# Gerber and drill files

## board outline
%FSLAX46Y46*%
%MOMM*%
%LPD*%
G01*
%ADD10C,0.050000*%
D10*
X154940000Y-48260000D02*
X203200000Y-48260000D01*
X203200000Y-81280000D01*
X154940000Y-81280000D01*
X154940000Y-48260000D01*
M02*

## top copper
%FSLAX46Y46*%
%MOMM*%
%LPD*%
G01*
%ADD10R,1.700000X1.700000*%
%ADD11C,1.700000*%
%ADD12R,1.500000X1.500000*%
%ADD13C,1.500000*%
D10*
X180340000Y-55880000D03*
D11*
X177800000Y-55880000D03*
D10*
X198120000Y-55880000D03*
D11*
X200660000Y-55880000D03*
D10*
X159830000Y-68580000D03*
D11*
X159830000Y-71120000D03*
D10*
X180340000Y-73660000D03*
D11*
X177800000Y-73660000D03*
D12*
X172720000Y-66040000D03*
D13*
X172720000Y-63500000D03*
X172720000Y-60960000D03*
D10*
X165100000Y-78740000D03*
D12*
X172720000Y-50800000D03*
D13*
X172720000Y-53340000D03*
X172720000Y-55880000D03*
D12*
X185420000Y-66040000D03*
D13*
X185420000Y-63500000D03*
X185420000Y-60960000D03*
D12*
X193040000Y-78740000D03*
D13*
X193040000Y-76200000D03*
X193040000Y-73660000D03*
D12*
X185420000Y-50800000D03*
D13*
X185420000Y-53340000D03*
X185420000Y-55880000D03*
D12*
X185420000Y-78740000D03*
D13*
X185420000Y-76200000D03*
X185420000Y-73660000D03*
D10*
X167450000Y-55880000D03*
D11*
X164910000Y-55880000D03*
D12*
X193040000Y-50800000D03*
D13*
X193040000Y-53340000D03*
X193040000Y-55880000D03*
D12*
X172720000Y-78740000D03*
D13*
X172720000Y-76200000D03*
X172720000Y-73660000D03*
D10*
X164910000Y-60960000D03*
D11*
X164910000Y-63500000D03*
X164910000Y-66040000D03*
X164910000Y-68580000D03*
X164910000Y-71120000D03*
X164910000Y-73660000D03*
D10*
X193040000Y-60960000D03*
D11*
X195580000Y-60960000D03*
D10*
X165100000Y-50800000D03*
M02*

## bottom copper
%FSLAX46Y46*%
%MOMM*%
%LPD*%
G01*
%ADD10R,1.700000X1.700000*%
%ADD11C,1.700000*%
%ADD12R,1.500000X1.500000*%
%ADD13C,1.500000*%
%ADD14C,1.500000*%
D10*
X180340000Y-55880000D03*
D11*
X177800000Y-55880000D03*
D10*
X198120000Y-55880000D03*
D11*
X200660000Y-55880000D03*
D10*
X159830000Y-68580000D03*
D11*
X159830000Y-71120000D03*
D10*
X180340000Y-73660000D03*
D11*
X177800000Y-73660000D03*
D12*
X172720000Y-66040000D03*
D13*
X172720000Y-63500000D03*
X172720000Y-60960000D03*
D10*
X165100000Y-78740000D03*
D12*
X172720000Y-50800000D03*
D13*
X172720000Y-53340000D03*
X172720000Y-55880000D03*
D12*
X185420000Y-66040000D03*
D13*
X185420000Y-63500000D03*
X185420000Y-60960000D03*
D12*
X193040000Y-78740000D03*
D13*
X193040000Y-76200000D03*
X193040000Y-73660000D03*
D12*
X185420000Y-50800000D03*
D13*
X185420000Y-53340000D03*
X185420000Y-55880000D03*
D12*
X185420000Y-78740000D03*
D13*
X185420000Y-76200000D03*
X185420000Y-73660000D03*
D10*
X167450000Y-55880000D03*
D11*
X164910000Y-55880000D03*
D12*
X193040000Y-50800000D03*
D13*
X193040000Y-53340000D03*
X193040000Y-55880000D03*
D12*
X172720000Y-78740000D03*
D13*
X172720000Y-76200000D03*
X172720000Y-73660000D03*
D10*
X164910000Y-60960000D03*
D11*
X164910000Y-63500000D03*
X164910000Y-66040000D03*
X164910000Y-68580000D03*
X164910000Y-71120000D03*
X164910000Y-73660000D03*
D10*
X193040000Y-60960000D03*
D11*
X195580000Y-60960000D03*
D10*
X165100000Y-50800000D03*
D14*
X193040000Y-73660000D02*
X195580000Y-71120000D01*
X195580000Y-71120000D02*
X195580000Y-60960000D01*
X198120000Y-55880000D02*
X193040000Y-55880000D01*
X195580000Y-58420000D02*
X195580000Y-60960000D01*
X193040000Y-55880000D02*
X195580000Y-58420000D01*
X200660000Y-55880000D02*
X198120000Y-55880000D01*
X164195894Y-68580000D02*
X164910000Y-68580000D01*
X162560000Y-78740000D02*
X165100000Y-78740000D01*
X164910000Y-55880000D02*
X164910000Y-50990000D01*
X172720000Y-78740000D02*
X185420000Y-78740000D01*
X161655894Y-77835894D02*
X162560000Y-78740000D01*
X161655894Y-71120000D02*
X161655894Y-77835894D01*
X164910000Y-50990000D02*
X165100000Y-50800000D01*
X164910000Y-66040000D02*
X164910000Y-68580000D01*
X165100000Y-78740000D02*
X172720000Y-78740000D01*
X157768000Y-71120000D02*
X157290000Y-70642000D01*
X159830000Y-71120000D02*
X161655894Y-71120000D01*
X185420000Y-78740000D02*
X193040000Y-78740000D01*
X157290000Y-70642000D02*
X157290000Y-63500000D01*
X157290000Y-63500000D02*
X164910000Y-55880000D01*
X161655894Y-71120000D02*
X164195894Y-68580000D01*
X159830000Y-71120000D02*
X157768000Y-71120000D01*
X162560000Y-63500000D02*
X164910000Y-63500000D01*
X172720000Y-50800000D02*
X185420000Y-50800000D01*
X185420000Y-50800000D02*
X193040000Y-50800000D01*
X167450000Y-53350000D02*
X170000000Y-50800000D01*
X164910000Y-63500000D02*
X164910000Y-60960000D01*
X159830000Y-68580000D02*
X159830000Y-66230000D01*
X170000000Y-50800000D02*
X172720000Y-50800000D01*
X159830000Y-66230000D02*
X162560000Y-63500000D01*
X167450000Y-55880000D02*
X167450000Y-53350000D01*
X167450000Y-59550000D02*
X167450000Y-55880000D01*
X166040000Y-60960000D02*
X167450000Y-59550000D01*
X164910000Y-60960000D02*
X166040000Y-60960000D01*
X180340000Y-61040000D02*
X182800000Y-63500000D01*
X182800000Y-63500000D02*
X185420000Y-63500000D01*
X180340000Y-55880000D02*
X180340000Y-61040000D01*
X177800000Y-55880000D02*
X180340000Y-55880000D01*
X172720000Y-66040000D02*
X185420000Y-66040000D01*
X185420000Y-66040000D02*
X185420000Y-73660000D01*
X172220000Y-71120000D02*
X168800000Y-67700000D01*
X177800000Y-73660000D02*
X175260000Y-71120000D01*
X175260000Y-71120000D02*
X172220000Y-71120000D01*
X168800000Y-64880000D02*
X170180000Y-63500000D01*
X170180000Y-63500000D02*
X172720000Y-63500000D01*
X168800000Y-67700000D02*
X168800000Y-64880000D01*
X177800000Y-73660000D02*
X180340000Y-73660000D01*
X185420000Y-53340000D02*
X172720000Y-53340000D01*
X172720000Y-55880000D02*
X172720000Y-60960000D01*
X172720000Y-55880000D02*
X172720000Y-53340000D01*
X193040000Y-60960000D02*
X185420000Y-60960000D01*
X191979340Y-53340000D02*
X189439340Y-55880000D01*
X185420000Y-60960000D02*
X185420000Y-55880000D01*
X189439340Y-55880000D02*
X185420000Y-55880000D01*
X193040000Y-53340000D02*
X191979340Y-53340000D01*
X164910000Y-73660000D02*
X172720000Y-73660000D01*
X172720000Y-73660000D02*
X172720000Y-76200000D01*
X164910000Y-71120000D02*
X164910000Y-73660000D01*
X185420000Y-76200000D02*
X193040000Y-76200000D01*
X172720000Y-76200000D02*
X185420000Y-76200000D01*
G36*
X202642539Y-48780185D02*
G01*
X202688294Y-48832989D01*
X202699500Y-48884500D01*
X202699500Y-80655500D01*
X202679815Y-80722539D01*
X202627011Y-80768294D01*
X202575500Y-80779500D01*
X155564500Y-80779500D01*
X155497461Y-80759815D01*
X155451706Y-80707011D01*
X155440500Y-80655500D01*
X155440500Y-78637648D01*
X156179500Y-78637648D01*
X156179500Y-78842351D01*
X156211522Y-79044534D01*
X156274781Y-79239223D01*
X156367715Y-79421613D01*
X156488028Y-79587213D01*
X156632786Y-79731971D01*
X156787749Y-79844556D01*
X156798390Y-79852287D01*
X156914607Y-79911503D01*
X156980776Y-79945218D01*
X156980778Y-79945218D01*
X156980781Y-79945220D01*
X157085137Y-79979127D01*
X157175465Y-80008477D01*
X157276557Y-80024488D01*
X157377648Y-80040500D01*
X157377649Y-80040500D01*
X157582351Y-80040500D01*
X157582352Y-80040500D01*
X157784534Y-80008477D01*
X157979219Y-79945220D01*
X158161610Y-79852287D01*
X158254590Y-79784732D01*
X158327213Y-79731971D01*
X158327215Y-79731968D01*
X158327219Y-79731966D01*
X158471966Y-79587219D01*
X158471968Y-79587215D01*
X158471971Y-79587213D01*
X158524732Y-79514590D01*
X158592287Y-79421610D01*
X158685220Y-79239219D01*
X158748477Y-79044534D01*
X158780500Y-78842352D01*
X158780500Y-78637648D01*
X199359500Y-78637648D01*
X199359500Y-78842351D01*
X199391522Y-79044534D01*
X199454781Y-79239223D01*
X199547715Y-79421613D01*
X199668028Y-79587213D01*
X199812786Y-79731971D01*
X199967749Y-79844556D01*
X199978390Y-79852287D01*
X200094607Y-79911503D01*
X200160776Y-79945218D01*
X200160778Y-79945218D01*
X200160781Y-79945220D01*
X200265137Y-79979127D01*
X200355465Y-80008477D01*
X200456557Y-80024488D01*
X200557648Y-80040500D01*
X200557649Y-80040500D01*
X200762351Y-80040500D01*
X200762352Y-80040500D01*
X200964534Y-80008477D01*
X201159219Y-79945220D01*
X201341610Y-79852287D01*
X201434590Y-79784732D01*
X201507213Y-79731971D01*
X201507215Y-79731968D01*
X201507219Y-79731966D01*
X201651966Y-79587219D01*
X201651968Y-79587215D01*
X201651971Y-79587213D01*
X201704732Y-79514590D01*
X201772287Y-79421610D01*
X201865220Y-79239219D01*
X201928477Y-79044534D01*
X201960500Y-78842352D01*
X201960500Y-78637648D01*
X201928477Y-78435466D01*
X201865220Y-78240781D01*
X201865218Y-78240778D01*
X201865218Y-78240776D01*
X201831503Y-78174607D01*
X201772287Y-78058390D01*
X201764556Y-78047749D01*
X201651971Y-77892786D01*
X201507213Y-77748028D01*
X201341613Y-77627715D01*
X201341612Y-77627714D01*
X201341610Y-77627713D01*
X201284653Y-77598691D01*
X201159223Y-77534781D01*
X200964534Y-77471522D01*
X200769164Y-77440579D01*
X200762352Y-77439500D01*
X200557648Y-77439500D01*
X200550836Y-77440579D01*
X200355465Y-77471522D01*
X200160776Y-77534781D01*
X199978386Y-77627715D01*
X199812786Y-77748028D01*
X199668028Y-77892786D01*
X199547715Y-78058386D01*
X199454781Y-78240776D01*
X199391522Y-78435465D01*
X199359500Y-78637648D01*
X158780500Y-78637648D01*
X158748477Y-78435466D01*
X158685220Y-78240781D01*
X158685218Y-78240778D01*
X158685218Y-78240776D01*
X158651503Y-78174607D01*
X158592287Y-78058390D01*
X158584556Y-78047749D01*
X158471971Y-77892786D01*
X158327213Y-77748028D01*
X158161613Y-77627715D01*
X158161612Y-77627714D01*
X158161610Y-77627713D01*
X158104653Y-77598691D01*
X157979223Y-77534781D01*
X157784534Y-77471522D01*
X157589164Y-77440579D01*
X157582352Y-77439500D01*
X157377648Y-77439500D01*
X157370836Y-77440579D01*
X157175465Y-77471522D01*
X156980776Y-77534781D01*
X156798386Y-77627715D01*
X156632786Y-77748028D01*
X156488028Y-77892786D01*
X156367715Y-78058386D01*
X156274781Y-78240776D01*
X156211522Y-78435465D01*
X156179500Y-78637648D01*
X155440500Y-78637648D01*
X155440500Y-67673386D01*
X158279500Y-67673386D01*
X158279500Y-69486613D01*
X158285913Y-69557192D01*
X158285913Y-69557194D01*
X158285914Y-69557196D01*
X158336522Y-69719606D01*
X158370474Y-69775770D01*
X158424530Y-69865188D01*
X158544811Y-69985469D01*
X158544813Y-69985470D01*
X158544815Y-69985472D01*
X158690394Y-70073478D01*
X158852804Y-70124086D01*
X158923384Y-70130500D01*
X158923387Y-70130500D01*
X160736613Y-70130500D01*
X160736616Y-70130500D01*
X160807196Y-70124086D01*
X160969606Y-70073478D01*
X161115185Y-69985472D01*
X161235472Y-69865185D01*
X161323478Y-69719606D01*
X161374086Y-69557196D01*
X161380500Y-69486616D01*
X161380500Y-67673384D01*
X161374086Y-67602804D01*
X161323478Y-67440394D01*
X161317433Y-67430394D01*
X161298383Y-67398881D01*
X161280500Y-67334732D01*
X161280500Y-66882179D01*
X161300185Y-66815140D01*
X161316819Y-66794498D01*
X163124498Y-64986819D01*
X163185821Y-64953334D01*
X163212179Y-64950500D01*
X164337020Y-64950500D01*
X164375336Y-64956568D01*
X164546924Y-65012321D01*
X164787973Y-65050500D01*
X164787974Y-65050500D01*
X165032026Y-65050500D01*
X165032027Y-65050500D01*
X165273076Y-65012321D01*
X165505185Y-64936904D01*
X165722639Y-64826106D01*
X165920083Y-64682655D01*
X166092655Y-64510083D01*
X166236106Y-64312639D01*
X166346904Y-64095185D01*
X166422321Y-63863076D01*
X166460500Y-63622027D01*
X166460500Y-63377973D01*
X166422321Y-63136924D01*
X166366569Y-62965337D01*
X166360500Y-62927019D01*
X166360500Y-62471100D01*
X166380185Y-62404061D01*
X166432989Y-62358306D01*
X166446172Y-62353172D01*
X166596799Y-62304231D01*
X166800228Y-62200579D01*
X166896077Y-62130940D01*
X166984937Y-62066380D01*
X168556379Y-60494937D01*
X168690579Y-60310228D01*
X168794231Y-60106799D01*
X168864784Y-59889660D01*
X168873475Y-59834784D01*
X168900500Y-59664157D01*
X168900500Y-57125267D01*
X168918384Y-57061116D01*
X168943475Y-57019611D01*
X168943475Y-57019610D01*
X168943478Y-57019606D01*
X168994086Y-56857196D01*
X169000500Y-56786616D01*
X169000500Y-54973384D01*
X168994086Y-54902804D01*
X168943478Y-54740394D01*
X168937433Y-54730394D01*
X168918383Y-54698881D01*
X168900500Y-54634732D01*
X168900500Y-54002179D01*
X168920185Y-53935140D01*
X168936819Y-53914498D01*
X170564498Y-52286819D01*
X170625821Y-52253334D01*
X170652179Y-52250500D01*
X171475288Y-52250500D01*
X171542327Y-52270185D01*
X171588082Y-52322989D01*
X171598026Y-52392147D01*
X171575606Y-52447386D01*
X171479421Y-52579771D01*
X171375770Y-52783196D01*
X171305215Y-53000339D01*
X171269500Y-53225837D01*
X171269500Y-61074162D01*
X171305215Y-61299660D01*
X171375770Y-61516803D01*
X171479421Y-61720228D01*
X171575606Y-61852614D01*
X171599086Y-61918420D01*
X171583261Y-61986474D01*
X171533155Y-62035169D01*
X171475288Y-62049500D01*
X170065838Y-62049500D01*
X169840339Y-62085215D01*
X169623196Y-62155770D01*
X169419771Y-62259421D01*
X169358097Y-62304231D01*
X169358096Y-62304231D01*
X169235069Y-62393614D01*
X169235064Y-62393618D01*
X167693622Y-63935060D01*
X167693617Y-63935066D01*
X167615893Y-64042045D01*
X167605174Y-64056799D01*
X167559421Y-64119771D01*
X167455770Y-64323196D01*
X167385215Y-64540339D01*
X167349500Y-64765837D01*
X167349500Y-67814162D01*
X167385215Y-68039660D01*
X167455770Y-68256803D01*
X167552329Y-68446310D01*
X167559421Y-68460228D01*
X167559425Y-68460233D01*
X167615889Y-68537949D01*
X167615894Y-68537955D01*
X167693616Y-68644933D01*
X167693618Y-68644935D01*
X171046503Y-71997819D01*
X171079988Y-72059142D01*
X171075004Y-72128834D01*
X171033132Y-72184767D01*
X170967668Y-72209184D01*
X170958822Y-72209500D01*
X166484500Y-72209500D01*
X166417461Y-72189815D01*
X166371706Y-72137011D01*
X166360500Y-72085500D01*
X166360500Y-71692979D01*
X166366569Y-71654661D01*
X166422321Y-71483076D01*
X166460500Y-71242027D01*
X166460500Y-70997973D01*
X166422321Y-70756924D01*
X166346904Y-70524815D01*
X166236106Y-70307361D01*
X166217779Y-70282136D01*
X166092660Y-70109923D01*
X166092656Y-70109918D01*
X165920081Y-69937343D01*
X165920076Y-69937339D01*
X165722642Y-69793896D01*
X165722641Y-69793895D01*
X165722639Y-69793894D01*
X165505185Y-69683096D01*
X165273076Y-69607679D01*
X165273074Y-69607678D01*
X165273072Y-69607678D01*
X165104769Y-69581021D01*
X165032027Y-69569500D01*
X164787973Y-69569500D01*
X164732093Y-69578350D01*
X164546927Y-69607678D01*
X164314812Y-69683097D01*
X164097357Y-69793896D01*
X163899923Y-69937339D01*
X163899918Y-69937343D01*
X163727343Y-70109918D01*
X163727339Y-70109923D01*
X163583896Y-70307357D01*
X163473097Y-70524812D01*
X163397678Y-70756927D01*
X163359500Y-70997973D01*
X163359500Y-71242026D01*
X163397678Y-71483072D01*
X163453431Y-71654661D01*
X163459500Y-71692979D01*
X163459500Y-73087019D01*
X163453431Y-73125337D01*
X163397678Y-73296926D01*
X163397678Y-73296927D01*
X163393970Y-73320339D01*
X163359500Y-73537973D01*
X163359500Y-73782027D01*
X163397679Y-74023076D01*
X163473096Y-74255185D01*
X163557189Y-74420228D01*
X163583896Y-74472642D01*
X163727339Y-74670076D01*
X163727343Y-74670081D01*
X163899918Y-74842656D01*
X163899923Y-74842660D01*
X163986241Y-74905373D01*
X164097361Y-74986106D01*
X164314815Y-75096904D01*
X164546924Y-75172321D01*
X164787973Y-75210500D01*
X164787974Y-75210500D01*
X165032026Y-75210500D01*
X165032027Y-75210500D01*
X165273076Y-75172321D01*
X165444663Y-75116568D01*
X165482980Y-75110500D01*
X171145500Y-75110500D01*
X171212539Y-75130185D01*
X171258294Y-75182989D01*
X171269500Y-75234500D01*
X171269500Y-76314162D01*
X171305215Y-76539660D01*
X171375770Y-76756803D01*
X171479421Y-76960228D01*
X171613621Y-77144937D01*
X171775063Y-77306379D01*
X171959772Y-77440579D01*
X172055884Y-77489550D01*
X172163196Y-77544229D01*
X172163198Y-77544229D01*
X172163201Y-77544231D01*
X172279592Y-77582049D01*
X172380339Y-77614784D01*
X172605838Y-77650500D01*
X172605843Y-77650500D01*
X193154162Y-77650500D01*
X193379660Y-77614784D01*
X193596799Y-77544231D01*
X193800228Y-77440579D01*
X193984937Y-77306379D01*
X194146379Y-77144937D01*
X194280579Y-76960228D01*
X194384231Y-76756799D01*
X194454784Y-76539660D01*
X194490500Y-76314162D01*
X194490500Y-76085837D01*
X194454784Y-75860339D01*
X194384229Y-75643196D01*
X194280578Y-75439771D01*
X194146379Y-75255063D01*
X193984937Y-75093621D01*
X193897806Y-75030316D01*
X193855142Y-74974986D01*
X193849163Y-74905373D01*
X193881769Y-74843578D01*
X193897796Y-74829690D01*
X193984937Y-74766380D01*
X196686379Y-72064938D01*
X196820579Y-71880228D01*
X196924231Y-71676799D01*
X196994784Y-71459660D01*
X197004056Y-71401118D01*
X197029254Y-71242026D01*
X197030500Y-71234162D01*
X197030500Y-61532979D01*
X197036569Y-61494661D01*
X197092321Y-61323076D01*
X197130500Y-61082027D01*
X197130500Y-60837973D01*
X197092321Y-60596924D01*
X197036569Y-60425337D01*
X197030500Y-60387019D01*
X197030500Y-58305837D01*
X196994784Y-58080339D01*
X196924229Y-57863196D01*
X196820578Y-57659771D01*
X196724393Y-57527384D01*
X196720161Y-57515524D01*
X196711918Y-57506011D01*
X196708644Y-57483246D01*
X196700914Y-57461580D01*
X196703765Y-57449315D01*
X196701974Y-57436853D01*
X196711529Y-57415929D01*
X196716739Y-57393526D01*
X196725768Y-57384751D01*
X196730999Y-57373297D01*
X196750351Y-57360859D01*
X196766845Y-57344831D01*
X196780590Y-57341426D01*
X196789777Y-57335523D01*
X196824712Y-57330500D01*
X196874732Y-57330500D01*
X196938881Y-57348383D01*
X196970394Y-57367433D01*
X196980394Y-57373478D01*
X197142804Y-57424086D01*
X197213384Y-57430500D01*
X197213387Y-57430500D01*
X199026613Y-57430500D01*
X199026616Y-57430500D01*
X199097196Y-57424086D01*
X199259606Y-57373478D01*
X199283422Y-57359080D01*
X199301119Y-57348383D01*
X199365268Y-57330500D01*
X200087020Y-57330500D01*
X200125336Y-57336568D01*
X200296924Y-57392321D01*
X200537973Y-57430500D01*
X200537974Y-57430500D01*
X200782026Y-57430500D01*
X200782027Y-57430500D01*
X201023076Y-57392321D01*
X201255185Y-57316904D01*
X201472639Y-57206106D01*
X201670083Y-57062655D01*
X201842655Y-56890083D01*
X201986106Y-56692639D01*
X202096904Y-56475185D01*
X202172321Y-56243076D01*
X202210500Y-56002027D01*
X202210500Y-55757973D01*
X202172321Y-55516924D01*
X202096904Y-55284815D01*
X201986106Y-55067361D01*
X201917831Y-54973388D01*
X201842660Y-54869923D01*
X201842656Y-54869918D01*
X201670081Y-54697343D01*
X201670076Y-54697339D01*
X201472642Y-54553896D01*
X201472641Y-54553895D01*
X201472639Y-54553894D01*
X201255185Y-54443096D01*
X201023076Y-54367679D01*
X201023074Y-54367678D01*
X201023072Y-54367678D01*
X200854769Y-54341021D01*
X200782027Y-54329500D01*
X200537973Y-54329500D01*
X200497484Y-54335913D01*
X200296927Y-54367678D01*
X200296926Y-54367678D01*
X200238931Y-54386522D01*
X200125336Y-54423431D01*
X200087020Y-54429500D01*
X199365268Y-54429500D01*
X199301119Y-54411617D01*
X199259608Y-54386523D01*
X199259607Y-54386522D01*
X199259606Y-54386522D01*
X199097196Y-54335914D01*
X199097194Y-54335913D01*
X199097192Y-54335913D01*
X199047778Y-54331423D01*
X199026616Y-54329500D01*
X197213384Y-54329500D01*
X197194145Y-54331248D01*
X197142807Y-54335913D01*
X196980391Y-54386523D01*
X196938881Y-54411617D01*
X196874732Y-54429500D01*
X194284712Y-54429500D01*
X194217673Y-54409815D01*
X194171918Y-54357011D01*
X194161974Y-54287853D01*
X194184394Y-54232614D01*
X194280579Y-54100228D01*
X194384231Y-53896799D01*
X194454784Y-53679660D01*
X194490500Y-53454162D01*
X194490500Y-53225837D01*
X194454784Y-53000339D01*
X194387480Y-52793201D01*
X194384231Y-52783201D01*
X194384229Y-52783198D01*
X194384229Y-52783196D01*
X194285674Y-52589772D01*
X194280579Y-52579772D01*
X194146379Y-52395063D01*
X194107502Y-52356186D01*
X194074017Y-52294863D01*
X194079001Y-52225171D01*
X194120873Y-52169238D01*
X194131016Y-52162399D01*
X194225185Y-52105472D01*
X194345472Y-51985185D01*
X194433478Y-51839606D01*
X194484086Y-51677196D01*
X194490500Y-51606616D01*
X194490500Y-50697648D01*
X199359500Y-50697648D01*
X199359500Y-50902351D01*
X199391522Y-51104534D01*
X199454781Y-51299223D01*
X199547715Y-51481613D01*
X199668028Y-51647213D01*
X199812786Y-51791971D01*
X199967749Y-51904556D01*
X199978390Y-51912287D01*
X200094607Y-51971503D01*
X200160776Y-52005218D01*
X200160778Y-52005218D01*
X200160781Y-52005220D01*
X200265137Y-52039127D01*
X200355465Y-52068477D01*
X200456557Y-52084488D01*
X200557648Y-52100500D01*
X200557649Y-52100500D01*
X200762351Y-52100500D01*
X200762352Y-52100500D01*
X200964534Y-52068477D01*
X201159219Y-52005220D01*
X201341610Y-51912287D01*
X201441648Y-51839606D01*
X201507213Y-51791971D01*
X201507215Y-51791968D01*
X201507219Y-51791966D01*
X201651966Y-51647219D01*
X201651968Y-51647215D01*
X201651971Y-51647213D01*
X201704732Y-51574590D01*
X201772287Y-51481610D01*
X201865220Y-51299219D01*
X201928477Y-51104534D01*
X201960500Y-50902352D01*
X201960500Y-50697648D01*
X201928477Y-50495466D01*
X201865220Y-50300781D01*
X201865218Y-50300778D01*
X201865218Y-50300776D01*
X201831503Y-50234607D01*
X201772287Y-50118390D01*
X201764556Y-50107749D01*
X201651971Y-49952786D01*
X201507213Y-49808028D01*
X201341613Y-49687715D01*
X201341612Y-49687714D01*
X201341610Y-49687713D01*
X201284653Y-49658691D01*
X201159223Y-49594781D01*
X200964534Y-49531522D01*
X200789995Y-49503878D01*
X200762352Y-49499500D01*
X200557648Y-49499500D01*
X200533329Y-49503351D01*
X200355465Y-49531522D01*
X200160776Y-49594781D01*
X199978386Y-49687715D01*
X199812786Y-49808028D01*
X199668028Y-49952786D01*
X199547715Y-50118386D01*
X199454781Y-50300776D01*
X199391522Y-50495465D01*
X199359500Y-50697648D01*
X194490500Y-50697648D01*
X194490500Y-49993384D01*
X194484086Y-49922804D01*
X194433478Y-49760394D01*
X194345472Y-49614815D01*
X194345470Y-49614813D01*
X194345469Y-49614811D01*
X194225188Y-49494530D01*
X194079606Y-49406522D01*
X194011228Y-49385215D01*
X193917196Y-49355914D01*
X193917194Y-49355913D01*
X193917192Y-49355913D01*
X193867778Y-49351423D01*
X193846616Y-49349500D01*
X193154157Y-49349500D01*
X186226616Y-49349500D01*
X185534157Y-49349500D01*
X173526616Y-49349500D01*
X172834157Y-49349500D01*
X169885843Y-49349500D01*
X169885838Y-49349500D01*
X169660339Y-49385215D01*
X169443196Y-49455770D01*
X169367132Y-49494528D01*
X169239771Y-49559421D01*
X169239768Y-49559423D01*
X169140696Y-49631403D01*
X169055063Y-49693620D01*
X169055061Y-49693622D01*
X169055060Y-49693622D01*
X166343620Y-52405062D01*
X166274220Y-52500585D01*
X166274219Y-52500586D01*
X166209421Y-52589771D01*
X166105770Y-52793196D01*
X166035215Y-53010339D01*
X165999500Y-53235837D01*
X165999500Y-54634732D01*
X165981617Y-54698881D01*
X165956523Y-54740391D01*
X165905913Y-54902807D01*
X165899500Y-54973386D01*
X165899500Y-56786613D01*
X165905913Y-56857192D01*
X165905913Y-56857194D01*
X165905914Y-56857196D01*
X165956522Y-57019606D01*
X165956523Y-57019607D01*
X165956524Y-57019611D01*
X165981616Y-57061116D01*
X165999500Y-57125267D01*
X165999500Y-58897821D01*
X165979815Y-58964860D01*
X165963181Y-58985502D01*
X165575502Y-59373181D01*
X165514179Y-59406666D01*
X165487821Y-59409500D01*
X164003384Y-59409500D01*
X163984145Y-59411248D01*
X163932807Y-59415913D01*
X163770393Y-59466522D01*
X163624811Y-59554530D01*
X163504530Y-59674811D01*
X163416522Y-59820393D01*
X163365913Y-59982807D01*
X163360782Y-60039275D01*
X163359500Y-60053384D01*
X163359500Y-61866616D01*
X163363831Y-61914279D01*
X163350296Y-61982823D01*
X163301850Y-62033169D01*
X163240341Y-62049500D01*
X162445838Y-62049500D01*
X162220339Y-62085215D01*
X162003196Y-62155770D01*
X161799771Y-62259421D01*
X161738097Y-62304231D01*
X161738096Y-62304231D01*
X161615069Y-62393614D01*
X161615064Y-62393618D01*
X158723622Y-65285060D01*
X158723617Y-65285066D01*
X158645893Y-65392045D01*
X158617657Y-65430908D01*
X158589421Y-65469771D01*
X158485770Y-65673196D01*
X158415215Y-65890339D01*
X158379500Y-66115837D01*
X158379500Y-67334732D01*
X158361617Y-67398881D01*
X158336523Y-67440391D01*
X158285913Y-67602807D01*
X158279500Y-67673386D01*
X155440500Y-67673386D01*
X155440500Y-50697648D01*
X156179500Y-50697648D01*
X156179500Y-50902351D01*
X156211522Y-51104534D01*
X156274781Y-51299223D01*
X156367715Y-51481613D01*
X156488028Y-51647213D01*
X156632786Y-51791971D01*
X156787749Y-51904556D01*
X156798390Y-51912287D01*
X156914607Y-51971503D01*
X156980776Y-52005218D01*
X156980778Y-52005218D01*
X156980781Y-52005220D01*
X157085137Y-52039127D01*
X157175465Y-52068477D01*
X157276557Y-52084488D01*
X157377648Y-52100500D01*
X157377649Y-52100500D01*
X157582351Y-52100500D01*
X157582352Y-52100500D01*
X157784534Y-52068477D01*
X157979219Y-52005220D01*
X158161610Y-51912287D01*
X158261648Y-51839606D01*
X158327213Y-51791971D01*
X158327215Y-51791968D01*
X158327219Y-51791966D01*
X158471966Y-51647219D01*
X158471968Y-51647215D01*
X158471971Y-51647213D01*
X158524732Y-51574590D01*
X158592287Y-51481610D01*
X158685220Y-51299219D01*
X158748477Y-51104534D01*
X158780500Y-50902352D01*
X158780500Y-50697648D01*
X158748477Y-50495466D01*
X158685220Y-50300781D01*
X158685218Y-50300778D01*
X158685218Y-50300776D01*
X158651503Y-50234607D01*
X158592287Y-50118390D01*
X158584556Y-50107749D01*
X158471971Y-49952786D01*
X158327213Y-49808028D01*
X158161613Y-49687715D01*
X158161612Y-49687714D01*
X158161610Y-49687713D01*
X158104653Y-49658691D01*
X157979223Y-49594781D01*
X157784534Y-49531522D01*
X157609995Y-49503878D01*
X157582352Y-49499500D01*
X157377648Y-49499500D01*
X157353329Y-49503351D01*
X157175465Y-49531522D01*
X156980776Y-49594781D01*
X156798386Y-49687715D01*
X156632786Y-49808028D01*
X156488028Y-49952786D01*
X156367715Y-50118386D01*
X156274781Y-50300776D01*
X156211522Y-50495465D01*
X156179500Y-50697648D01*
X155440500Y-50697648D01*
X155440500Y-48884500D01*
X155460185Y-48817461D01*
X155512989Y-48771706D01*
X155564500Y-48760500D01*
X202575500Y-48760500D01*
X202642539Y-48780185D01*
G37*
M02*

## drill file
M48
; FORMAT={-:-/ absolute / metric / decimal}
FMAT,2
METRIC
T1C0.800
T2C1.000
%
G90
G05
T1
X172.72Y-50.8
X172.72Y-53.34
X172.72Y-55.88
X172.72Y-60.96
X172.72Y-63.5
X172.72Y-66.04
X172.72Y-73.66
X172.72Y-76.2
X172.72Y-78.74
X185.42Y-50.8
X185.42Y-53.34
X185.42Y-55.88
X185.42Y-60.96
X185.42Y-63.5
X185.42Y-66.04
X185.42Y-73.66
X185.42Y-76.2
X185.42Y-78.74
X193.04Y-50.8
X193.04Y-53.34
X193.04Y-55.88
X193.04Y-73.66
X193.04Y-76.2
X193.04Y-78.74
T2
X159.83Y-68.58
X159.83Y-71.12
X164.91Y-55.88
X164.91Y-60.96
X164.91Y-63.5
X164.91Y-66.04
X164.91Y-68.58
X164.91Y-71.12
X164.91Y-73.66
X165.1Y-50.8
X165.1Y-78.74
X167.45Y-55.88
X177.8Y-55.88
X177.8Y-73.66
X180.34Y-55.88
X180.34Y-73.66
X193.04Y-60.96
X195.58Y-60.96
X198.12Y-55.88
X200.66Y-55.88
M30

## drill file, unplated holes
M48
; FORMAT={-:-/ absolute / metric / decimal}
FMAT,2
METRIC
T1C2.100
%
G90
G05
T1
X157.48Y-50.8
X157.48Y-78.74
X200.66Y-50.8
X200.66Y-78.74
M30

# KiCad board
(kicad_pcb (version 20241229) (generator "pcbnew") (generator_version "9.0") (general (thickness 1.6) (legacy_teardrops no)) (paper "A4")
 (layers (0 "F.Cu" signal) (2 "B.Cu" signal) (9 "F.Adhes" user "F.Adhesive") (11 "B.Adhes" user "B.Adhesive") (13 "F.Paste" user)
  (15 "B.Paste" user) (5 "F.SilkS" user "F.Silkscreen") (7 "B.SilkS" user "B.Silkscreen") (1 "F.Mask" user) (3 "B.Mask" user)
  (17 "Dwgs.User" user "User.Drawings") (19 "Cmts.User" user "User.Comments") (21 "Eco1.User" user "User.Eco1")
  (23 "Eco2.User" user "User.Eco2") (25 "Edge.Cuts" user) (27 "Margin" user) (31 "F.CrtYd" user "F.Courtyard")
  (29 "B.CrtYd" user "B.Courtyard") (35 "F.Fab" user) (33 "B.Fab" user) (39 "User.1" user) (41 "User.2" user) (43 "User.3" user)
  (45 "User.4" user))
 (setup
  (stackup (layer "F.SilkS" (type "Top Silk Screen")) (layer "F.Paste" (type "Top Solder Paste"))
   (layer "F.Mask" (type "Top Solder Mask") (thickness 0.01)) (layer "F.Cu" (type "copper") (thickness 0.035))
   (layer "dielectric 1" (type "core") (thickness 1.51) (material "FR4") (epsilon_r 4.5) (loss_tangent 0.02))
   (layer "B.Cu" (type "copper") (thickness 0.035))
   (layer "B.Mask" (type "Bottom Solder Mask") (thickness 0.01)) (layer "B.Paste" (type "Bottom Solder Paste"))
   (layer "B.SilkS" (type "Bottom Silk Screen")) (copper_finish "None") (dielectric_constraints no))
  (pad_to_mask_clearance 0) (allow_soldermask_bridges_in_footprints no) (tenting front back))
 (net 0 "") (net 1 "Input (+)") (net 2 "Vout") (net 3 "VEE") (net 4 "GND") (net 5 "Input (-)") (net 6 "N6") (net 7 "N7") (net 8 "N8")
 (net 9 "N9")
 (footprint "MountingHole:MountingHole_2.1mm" (layer "F.Cu") (at 157.48 78.74)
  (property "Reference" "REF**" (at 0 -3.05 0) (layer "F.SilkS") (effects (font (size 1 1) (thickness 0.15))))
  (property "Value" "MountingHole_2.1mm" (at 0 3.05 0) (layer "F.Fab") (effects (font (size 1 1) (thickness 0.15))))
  (pad "" np_thru_hole circle (at 0 0) (size 2.1 2.1) (drill 2.1) (layers "*.Cu" "*.Mask")))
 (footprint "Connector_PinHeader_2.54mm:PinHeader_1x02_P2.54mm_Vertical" (layer "F.Cu") (at 180.34 55.88 -90)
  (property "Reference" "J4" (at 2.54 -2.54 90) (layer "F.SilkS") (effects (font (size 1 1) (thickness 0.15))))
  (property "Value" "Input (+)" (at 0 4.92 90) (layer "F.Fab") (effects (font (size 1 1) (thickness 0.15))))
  (pad "1" thru_hole rect (at 0 0 270) (size 1.7 1.7) (drill 1) (layers "*.Cu" "*.Mask") (remove_unused_layers no) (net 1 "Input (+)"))
  (pad "2" thru_hole circle (at 0 2.54 270) (size 1.7 1.7) (drill 1) (layers "*.Cu" "*.Mask") (remove_unused_layers no) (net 1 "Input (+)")))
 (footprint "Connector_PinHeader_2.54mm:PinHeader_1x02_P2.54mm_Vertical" (layer "F.Cu") (at 198.12 55.88 90)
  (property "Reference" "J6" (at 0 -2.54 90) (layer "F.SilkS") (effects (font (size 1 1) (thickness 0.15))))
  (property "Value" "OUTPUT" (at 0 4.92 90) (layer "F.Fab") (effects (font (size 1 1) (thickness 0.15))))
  (pad "1" thru_hole rect (at 0 0 90) (size 1.7 1.7) (drill 1) (layers "*.Cu" "*.Mask") (remove_unused_layers no) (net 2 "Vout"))
  (pad "2" thru_hole circle (at 0 2.54 90) (size 1.7 1.7) (drill 1) (layers "*.Cu" "*.Mask") (remove_unused_layers no) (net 2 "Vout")))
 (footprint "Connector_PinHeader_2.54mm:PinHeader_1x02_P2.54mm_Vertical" (layer "F.Cu") (at 159.83 68.58)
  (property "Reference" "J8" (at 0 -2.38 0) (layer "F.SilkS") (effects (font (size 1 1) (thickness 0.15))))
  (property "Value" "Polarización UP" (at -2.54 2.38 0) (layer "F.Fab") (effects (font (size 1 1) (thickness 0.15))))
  (pad "1" thru_hole rect (at 0 0) (size 1.7 1.7) (drill 1) (layers "*.Cu" "*.Mask") (remove_unused_layers no) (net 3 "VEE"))
  (pad "2" thru_hole circle (at 0 2.54) (size 1.7 1.7) (drill 1) (layers "*.Cu" "*.Mask") (remove_unused_layers no) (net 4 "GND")))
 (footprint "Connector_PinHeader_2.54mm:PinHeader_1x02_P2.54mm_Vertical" (layer "F.Cu") (at 180.34 73.66 -90)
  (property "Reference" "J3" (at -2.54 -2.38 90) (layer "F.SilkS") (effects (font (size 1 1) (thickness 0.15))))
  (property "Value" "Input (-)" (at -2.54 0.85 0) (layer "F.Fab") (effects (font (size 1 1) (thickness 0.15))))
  (pad "1" thru_hole rect (at 0 0 270) (size 1.7 1.7) (drill 1) (layers "*.Cu" "*.Mask") (remove_unused_layers no) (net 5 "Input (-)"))
  (pad "2" thru_hole circle (at 0 2.54 270) (size 1.7 1.7) (drill 1) (layers "*.Cu" "*.Mask") (remove_unused_layers no) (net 5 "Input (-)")))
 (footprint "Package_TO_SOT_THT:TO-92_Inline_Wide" (layer "F.Cu") (at 172.72 66.04 90)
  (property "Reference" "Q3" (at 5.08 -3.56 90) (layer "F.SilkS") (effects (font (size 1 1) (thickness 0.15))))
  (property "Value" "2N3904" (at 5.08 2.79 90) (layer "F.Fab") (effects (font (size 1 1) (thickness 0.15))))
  (pad "1" thru_hole rect (at 0 0 90) (size 1.5 1.5) (drill 0.8) (layers "*.Cu" "*.Mask") (remove_unused_layers no) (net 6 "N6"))
  (pad "2" thru_hole circle (at 2.54 0 90) (size 1.5 1.5) (drill 0.8) (layers "*.Cu" "*.Mask") (remove_unused_layers no) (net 5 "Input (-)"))
  (pad "3" thru_hole circle (at 5.08 0 90) (size 1.5 1.5) (drill 0.8) (layers "*.Cu" "*.Mask") (remove_unused_layers no) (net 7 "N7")))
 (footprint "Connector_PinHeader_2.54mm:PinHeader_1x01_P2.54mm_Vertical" (layer "F.Cu") (at 165.1 78.74)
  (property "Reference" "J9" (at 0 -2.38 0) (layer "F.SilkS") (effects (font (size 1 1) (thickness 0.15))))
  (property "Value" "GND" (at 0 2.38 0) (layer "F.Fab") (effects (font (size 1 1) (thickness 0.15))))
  (pad "1" thru_hole rect (at 0 0) (size 1.7 1.7) (drill 1) (layers "*.Cu" "*.Mask") (remove_unused_layers no) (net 4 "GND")))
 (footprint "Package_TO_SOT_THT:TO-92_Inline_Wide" (layer "F.Cu") (at 172.72 50.8 -90)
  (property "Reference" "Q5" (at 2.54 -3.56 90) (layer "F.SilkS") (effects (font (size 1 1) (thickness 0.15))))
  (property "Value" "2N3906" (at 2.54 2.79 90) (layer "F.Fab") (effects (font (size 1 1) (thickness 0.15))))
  (pad "1" thru_hole rect (at 0 0 270) (size 1.5 1.5) (drill 0.8) (layers "*.Cu" "*.Mask") (remove_unused_layers no) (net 3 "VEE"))
  (pad "2" thru_hole circle (at 2.54 0 270) (size 1.5 1.5) (drill 0.8) (layers "*.Cu" "*.Mask") (remove_unused_layers no) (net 7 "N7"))
  (pad "3" thru_hole circle (at 5.08 0 270) (size 1.5 1.5) (drill 0.8) (layers "*.Cu" "*.Mask") (remove_unused_layers no) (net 7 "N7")))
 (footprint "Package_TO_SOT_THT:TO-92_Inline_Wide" (layer "F.Cu") (at 185.42 66.04 90)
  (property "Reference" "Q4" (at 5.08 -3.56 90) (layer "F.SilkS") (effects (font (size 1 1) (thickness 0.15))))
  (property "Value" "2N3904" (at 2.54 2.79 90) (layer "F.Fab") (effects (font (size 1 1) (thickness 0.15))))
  (pad "1" thru_hole rect (at 0 0 90) (size 1.5 1.5) (drill 0.8) (layers "*.Cu" "*.Mask") (remove_unused_layers no) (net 6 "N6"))
  (pad "2" thru_hole circle (at 2.54 0 90) (size 1.5 1.5) (drill 0.8) (layers "*.Cu" "*.Mask") (remove_unused_layers no) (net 1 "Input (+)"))
  (pad "3" thru_hole circle (at 5.08 0 90) (size 1.5 1.5) (drill 0.8) (layers "*.Cu" "*.Mask") (remove_unused_layers no) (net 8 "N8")))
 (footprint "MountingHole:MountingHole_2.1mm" (layer "F.Cu") (at 200.66 78.74)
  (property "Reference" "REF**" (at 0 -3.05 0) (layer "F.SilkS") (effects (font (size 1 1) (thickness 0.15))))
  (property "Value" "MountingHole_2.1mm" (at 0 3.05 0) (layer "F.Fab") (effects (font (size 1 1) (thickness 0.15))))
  (pad "" np_thru_hole circle (at 0 0) (size 2.1 2.1) (drill 2.1) (layers "*.Cu" "*.Mask")))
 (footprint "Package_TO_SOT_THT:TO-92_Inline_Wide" (layer "F.Cu") (at 193.04 78.74 90)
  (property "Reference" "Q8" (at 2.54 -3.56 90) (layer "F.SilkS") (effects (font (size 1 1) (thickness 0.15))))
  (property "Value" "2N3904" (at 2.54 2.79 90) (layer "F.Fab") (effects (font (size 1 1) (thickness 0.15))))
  (pad "1" thru_hole rect (at 0 0 90) (size 1.5 1.5) (drill 0.8) (layers "*.Cu" "*.Mask") (remove_unused_layers no) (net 4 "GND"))
  (pad "2" thru_hole circle (at 2.54 0 90) (size 1.5 1.5) (drill 0.8) (layers "*.Cu" "*.Mask") (remove_unused_layers no) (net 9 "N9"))
  (pad "3" thru_hole circle (at 5.08 0 90) (size 1.5 1.5) (drill 0.8) (layers "*.Cu" "*.Mask") (remove_unused_layers no) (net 2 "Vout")))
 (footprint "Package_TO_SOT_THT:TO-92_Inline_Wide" (layer "F.Cu") (at 185.42 50.8 -90)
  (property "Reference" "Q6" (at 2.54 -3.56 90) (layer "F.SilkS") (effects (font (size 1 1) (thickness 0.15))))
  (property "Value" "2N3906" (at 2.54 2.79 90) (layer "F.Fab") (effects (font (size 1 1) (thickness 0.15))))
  (pad "1" thru_hole rect (at 0 0 270) (size 1.5 1.5) (drill 0.8) (layers "*.Cu" "*.Mask") (remove_unused_layers no) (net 3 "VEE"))
  (pad "2" thru_hole circle (at 2.54 0 270) (size 1.5 1.5) (drill 0.8) (layers "*.Cu" "*.Mask") (remove_unused_layers no) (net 7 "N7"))
  (pad "3" thru_hole circle (at 5.08 0 270) (size 1.5 1.5) (drill 0.8) (layers "*.Cu" "*.Mask") (remove_unused_layers no) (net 8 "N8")))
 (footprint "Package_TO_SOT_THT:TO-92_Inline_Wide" (layer "F.Cu") (at 185.42 78.74 90)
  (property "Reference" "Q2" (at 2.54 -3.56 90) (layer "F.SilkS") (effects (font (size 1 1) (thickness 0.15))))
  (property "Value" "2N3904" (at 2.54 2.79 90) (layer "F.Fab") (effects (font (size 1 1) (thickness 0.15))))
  (pad "1" thru_hole rect (at 0 0 90) (size 1.5 1.5) (drill 0.8) (layers "*.Cu" "*.Mask") (remove_unused_layers no) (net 4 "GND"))
  (pad "2" thru_hole circle (at 2.54 0 90) (size 1.5 1.5) (drill 0.8) (layers "*.Cu" "*.Mask") (remove_unused_layers no) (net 9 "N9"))
  (pad "3" thru_hole circle (at 5.08 0 90) (size 1.5 1.5) (drill 0.8) (layers "*.Cu" "*.Mask") (remove_unused_layers no) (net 6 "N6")))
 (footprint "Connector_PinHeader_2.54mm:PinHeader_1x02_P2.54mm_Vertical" (layer "F.Cu") (at 167.45 55.88 -90)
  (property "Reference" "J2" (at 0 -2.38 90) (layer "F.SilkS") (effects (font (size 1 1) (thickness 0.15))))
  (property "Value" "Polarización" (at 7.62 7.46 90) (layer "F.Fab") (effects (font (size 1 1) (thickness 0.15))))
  (pad "1" thru_hole rect (at 0 0 270) (size 1.7 1.7) (drill 1) (layers "*.Cu" "*.Mask") (remove_unused_layers no) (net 3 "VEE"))
  (pad "2" thru_hole circle (at 0 2.54 270) (size 1.7 1.7) (drill 1) (layers "*.Cu" "*.Mask") (remove_unused_layers no) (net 4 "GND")))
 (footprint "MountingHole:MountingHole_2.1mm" (layer "F.Cu") (at 157.48 50.8)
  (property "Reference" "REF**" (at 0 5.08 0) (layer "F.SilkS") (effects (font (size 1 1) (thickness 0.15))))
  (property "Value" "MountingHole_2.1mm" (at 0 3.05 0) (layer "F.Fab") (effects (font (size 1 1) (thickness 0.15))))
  (pad "" np_thru_hole circle (at 0 0) (size 2.1 2.1) (drill 2.1) (layers "*.Cu" "*.Mask")))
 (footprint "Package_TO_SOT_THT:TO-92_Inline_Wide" (layer "F.Cu") (at 193.04 50.8 -90)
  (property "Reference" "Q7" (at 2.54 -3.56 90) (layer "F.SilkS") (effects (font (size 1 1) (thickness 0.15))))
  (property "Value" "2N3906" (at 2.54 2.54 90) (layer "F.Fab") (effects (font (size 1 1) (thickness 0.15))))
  (pad "1" thru_hole rect (at 0 0 270) (size 1.5 1.5) (drill 0.8) (layers "*.Cu" "*.Mask") (remove_unused_layers no) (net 3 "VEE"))
  (pad "2" thru_hole circle (at 2.54 0 270) (size 1.5 1.5) (drill 0.8) (layers "*.Cu" "*.Mask") (remove_unused_layers no) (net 8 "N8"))
  (pad "3" thru_hole circle (at 5.08 0 270) (size 1.5 1.5) (drill 0.8) (layers "*.Cu" "*.Mask") (remove_unused_layers no) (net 2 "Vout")))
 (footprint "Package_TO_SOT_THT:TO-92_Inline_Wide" (layer "F.Cu") (at 172.72 78.74 90)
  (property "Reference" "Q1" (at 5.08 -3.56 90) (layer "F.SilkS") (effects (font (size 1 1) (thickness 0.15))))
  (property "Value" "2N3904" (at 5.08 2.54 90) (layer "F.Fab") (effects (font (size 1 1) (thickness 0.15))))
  (pad "1" thru_hole rect (at 0 0 90) (size 1.5 1.5) (drill 0.8) (layers "*.Cu" "*.Mask") (remove_unused_layers no) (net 4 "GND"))
  (pad "2" thru_hole circle (at 2.54 0 90) (size 1.5 1.5) (drill 0.8) (layers "*.Cu" "*.Mask") (remove_unused_layers no) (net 9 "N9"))
  (pad "3" thru_hole circle (at 5.08 0 90) (size 1.5 1.5) (drill 0.8) (layers "*.Cu" "*.Mask") (remove_unused_layers no) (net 9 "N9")))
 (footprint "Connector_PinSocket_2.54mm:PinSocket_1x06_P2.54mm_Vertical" (layer "F.Cu") (at 164.91 60.96)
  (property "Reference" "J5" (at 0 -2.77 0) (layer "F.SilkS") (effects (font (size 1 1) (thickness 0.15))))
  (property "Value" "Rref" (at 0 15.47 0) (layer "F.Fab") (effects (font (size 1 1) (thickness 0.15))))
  (pad "1" thru_hole rect (at 0 0) (size 1.7 1.7) (drill 1) (layers "*.Cu" "*.Mask") (remove_unused_layers no) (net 3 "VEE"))
  (pad "2" thru_hole circle (at 0 2.54) (size 1.7 1.7) (drill 1) (layers "*.Cu" "*.Mask") (remove_unused_layers no) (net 3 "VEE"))
  (pad "3" thru_hole circle (at 0 5.08) (size 1.7 1.7) (drill 1) (layers "*.Cu" "*.Mask") (remove_unused_layers no) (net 4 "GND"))
  (pad "4" thru_hole circle (at 0 7.62) (size 1.7 1.7) (drill 1) (layers "*.Cu" "*.Mask") (remove_unused_layers no) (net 4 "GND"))
  (pad "5" thru_hole circle (at 0 10.16) (size 1.7 1.7) (drill 1) (layers "*.Cu" "*.Mask") (remove_unused_layers no) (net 9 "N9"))
  (pad "6" thru_hole circle (at 0 12.7) (size 1.7 1.7) (drill 1) (layers "*.Cu" "*.Mask") (remove_unused_layers no) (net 9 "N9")))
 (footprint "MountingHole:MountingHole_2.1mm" (layer "F.Cu") (at 200.66 50.8)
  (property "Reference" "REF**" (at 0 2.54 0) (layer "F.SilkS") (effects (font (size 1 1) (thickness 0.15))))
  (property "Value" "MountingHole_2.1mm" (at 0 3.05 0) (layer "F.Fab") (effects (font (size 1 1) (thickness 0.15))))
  (pad "" np_thru_hole circle (at 0 0) (size 2.1 2.1) (drill 2.1) (layers "*.Cu" "*.Mask")))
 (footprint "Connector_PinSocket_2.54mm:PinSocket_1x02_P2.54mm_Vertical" (layer "F.Cu") (at 193.04 60.96 90)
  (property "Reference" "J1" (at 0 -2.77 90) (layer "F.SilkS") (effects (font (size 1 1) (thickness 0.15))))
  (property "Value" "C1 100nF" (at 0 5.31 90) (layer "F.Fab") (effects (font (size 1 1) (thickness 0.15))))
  (pad "1" thru_hole rect (at 0 0 90) (size 1.7 1.7) (drill 1) (layers "*.Cu" "*.Mask") (remove_unused_layers no) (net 8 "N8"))
  (pad "2" thru_hole circle (at 0 2.54 90) (size 1.7 1.7) (drill 1) (layers "*.Cu" "*.Mask") (remove_unused_layers no) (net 2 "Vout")))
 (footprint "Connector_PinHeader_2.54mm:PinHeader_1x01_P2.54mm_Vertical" (layer "F.Cu") (at 165.1 50.8)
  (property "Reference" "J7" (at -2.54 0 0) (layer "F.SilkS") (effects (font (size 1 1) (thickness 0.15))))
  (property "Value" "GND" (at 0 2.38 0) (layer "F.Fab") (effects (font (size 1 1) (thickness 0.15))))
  (pad "1" thru_hole rect (at 0 0) (size 1.7 1.7) (drill 1) (layers "*.Cu" "*.Mask") (remove_unused_layers no) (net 4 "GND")))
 (gr_rect (start 154.94 48.26) (end 203.2 81.28) (stroke (width 0.05) (type default)) (fill no) (layer "Edge.Cuts"))
 (segment (start 193.04 73.66) (end 195.58 71.12) (width 1.5) (layer "B.Cu") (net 2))
 (segment (start 195.58 71.12) (end 195.58 60.96) (width 1.5) (layer "B.Cu") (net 2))
 (segment (start 198.12 55.88) (end 193.04 55.88) (width 1.5) (layer "B.Cu") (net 2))
 (segment (start 195.58 58.42) (end 195.58 60.96) (width 1.5) (layer "B.Cu") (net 2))
 (segment (start 193.04 55.88) (end 195.58 58.42) (width 1.5) (layer "B.Cu") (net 2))
 (segment (start 200.66 55.88) (end 198.12 55.88) (width 1.5) (layer "B.Cu") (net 2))
 (segment (start 164.195894 68.58) (end 164.91 68.58) (width 1.5) (layer "B.Cu") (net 4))
 (segment (start 162.56 78.74) (end 165.1 78.74) (width 1.5) (layer "B.Cu") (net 4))
 (segment (start 164.91 55.88) (end 164.91 50.99) (width 1.5) (layer "B.Cu") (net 4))
 (segment (start 172.72 78.74) (end 185.42 78.74) (width 1.5) (layer "B.Cu") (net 4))
 (segment (start 161.655894 77.835894) (end 162.56 78.74) (width 1.5) (layer "B.Cu") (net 4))
 (segment (start 161.655894 71.12) (end 161.655894 77.835894) (width 1.5) (layer "B.Cu") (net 4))
 (segment (start 164.91 50.99) (end 165.1 50.8) (width 1.5) (layer "B.Cu") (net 4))
 (segment (start 164.91 66.04) (end 164.91 68.58) (width 1.5) (layer "B.Cu") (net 4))
 (segment (start 165.1 78.74) (end 172.72 78.74) (width 1.5) (layer "B.Cu") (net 4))
 (segment (start 157.768 71.12) (end 157.29 70.642) (width 1.5) (layer "B.Cu") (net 4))
 (segment (start 159.83 71.12) (end 161.655894 71.12) (width 1.5) (layer "B.Cu") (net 4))
 (segment (start 185.42 78.74) (end 193.04 78.74) (width 1.5) (layer "B.Cu") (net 4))
 (segment (start 157.29 70.642) (end 157.29 63.5) (width 1.5) (layer "B.Cu") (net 4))
 (segment (start 157.29 63.5) (end 164.91 55.88) (width 1.5) (layer "B.Cu") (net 4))
 (segment (start 161.655894 71.12) (end 164.195894 68.58) (width 1.5) (layer "B.Cu") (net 4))
 (segment (start 159.83 71.12) (end 157.768 71.12) (width 1.5) (layer "B.Cu") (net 4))
 (segment (start 162.56 63.5) (end 164.91 63.5) (width 1.5) (layer "B.Cu") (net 3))
 (segment (start 172.72 50.8) (end 185.42 50.8) (width 1.5) (layer "B.Cu") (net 3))
 (segment (start 185.42 50.8) (end 193.04 50.8) (width 1.5) (layer "B.Cu") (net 3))
 (segment (start 167.45 53.35) (end 170 50.8) (width 1.5) (layer "B.Cu") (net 3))
 (segment (start 164.91 63.5) (end 164.91 60.96) (width 1.5) (layer "B.Cu") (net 3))
 (segment (start 159.83 68.58) (end 159.83 66.23) (width 1.5) (layer "B.Cu") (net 3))
 (segment (start 170 50.8) (end 172.72 50.8) (width 1.5) (layer "B.Cu") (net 3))
 (segment (start 159.83 66.23) (end 162.56 63.5) (width 1.5) (layer "B.Cu") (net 3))
 (segment (start 167.45 55.88) (end 167.45 53.35) (width 1.5) (layer "B.Cu") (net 3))
 (segment (start 167.45 59.55) (end 167.45 55.88) (width 1.5) (layer "B.Cu") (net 3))
 (segment (start 166.04 60.96) (end 167.45 59.55) (width 1.5) (layer "B.Cu") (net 3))
 (segment (start 164.91 60.96) (end 166.04 60.96) (width 1.5) (layer "B.Cu") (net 3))
 (segment (start 180.34 61.04) (end 182.8 63.5) (width 1.5) (layer "B.Cu") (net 1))
 (segment (start 182.8 63.5) (end 185.42 63.5) (width 1.5) (layer "B.Cu") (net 1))
 (segment (start 180.34 55.88) (end 180.34 61.04) (width 1.5) (layer "B.Cu") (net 1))
 (segment (start 177.8 55.88) (end 180.34 55.88) (width 1.5) (layer "B.Cu") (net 1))
 (segment (start 172.72 66.04) (end 185.42 66.04) (width 1.5) (layer "B.Cu") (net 6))
 (segment (start 185.42 66.04) (end 185.42 73.66) (width 1.5) (layer "B.Cu") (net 6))
 (segment (start 172.22 71.12) (end 168.8 67.7) (width 1.5) (layer "B.Cu") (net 5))
 (segment (start 177.8 73.66) (end 175.26 71.12) (width 1.5) (layer "B.Cu") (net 5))
 (segment (start 175.26 71.12) (end 172.22 71.12) (width 1.5) (layer "B.Cu") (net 5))
 (segment (start 168.8 64.88) (end 170.18 63.5) (width 1.5) (layer "B.Cu") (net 5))
 (segment (start 170.18 63.5) (end 172.72 63.5) (width 1.5) (layer "B.Cu") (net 5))
 (segment (start 168.8 67.7) (end 168.8 64.88) (width 1.5) (layer "B.Cu") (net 5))
 (segment (start 177.8 73.66) (end 180.34 73.66) (width 1.5) (layer "B.Cu") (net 5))
 (segment (start 185.42 53.34) (end 172.72 53.34) (width 1.5) (layer "B.Cu") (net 7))
 (segment (start 172.72 55.88) (end 172.72 60.96) (width 1.5) (layer "B.Cu") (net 7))
 (segment (start 172.72 55.88) (end 172.72 53.34) (width 1.5) (layer "B.Cu") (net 7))
 (segment (start 193.04 60.96) (end 185.42 60.96) (width 1.5) (layer "B.Cu") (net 8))
 (segment (start 191.97934 53.34) (end 189.43934 55.88) (width 1.5) (layer "B.Cu") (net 8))
 (segment (start 185.42 60.96) (end 185.42 55.88) (width 1.5) (layer "B.Cu") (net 8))
 (segment (start 189.43934 55.88) (end 185.42 55.88) (width 1.5) (layer "B.Cu") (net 8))
 (segment (start 193.04 53.34) (end 191.97934 53.34) (width 1.5) (layer "B.Cu") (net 8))
 (segment (start 164.91 73.66) (end 172.72 73.66) (width 1.5) (layer "B.Cu") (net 9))
 (segment (start 172.72 73.66) (end 172.72 76.2) (width 1.5) (layer "B.Cu") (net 9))
 (segment (start 164.91 71.12) (end 164.91 73.66) (width 1.5) (layer "B.Cu") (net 9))
 (segment (start 185.42 76.2) (end 193.04 76.2) (width 1.5) (layer "B.Cu") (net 9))
 (segment (start 172.72 76.2) (end 185.42 76.2) (width 1.5) (layer "B.Cu") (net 9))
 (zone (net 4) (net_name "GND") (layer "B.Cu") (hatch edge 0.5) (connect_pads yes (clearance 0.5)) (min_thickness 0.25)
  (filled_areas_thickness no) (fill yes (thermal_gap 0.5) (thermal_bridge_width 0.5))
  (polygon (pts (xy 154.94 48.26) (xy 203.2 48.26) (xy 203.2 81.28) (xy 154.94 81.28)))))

